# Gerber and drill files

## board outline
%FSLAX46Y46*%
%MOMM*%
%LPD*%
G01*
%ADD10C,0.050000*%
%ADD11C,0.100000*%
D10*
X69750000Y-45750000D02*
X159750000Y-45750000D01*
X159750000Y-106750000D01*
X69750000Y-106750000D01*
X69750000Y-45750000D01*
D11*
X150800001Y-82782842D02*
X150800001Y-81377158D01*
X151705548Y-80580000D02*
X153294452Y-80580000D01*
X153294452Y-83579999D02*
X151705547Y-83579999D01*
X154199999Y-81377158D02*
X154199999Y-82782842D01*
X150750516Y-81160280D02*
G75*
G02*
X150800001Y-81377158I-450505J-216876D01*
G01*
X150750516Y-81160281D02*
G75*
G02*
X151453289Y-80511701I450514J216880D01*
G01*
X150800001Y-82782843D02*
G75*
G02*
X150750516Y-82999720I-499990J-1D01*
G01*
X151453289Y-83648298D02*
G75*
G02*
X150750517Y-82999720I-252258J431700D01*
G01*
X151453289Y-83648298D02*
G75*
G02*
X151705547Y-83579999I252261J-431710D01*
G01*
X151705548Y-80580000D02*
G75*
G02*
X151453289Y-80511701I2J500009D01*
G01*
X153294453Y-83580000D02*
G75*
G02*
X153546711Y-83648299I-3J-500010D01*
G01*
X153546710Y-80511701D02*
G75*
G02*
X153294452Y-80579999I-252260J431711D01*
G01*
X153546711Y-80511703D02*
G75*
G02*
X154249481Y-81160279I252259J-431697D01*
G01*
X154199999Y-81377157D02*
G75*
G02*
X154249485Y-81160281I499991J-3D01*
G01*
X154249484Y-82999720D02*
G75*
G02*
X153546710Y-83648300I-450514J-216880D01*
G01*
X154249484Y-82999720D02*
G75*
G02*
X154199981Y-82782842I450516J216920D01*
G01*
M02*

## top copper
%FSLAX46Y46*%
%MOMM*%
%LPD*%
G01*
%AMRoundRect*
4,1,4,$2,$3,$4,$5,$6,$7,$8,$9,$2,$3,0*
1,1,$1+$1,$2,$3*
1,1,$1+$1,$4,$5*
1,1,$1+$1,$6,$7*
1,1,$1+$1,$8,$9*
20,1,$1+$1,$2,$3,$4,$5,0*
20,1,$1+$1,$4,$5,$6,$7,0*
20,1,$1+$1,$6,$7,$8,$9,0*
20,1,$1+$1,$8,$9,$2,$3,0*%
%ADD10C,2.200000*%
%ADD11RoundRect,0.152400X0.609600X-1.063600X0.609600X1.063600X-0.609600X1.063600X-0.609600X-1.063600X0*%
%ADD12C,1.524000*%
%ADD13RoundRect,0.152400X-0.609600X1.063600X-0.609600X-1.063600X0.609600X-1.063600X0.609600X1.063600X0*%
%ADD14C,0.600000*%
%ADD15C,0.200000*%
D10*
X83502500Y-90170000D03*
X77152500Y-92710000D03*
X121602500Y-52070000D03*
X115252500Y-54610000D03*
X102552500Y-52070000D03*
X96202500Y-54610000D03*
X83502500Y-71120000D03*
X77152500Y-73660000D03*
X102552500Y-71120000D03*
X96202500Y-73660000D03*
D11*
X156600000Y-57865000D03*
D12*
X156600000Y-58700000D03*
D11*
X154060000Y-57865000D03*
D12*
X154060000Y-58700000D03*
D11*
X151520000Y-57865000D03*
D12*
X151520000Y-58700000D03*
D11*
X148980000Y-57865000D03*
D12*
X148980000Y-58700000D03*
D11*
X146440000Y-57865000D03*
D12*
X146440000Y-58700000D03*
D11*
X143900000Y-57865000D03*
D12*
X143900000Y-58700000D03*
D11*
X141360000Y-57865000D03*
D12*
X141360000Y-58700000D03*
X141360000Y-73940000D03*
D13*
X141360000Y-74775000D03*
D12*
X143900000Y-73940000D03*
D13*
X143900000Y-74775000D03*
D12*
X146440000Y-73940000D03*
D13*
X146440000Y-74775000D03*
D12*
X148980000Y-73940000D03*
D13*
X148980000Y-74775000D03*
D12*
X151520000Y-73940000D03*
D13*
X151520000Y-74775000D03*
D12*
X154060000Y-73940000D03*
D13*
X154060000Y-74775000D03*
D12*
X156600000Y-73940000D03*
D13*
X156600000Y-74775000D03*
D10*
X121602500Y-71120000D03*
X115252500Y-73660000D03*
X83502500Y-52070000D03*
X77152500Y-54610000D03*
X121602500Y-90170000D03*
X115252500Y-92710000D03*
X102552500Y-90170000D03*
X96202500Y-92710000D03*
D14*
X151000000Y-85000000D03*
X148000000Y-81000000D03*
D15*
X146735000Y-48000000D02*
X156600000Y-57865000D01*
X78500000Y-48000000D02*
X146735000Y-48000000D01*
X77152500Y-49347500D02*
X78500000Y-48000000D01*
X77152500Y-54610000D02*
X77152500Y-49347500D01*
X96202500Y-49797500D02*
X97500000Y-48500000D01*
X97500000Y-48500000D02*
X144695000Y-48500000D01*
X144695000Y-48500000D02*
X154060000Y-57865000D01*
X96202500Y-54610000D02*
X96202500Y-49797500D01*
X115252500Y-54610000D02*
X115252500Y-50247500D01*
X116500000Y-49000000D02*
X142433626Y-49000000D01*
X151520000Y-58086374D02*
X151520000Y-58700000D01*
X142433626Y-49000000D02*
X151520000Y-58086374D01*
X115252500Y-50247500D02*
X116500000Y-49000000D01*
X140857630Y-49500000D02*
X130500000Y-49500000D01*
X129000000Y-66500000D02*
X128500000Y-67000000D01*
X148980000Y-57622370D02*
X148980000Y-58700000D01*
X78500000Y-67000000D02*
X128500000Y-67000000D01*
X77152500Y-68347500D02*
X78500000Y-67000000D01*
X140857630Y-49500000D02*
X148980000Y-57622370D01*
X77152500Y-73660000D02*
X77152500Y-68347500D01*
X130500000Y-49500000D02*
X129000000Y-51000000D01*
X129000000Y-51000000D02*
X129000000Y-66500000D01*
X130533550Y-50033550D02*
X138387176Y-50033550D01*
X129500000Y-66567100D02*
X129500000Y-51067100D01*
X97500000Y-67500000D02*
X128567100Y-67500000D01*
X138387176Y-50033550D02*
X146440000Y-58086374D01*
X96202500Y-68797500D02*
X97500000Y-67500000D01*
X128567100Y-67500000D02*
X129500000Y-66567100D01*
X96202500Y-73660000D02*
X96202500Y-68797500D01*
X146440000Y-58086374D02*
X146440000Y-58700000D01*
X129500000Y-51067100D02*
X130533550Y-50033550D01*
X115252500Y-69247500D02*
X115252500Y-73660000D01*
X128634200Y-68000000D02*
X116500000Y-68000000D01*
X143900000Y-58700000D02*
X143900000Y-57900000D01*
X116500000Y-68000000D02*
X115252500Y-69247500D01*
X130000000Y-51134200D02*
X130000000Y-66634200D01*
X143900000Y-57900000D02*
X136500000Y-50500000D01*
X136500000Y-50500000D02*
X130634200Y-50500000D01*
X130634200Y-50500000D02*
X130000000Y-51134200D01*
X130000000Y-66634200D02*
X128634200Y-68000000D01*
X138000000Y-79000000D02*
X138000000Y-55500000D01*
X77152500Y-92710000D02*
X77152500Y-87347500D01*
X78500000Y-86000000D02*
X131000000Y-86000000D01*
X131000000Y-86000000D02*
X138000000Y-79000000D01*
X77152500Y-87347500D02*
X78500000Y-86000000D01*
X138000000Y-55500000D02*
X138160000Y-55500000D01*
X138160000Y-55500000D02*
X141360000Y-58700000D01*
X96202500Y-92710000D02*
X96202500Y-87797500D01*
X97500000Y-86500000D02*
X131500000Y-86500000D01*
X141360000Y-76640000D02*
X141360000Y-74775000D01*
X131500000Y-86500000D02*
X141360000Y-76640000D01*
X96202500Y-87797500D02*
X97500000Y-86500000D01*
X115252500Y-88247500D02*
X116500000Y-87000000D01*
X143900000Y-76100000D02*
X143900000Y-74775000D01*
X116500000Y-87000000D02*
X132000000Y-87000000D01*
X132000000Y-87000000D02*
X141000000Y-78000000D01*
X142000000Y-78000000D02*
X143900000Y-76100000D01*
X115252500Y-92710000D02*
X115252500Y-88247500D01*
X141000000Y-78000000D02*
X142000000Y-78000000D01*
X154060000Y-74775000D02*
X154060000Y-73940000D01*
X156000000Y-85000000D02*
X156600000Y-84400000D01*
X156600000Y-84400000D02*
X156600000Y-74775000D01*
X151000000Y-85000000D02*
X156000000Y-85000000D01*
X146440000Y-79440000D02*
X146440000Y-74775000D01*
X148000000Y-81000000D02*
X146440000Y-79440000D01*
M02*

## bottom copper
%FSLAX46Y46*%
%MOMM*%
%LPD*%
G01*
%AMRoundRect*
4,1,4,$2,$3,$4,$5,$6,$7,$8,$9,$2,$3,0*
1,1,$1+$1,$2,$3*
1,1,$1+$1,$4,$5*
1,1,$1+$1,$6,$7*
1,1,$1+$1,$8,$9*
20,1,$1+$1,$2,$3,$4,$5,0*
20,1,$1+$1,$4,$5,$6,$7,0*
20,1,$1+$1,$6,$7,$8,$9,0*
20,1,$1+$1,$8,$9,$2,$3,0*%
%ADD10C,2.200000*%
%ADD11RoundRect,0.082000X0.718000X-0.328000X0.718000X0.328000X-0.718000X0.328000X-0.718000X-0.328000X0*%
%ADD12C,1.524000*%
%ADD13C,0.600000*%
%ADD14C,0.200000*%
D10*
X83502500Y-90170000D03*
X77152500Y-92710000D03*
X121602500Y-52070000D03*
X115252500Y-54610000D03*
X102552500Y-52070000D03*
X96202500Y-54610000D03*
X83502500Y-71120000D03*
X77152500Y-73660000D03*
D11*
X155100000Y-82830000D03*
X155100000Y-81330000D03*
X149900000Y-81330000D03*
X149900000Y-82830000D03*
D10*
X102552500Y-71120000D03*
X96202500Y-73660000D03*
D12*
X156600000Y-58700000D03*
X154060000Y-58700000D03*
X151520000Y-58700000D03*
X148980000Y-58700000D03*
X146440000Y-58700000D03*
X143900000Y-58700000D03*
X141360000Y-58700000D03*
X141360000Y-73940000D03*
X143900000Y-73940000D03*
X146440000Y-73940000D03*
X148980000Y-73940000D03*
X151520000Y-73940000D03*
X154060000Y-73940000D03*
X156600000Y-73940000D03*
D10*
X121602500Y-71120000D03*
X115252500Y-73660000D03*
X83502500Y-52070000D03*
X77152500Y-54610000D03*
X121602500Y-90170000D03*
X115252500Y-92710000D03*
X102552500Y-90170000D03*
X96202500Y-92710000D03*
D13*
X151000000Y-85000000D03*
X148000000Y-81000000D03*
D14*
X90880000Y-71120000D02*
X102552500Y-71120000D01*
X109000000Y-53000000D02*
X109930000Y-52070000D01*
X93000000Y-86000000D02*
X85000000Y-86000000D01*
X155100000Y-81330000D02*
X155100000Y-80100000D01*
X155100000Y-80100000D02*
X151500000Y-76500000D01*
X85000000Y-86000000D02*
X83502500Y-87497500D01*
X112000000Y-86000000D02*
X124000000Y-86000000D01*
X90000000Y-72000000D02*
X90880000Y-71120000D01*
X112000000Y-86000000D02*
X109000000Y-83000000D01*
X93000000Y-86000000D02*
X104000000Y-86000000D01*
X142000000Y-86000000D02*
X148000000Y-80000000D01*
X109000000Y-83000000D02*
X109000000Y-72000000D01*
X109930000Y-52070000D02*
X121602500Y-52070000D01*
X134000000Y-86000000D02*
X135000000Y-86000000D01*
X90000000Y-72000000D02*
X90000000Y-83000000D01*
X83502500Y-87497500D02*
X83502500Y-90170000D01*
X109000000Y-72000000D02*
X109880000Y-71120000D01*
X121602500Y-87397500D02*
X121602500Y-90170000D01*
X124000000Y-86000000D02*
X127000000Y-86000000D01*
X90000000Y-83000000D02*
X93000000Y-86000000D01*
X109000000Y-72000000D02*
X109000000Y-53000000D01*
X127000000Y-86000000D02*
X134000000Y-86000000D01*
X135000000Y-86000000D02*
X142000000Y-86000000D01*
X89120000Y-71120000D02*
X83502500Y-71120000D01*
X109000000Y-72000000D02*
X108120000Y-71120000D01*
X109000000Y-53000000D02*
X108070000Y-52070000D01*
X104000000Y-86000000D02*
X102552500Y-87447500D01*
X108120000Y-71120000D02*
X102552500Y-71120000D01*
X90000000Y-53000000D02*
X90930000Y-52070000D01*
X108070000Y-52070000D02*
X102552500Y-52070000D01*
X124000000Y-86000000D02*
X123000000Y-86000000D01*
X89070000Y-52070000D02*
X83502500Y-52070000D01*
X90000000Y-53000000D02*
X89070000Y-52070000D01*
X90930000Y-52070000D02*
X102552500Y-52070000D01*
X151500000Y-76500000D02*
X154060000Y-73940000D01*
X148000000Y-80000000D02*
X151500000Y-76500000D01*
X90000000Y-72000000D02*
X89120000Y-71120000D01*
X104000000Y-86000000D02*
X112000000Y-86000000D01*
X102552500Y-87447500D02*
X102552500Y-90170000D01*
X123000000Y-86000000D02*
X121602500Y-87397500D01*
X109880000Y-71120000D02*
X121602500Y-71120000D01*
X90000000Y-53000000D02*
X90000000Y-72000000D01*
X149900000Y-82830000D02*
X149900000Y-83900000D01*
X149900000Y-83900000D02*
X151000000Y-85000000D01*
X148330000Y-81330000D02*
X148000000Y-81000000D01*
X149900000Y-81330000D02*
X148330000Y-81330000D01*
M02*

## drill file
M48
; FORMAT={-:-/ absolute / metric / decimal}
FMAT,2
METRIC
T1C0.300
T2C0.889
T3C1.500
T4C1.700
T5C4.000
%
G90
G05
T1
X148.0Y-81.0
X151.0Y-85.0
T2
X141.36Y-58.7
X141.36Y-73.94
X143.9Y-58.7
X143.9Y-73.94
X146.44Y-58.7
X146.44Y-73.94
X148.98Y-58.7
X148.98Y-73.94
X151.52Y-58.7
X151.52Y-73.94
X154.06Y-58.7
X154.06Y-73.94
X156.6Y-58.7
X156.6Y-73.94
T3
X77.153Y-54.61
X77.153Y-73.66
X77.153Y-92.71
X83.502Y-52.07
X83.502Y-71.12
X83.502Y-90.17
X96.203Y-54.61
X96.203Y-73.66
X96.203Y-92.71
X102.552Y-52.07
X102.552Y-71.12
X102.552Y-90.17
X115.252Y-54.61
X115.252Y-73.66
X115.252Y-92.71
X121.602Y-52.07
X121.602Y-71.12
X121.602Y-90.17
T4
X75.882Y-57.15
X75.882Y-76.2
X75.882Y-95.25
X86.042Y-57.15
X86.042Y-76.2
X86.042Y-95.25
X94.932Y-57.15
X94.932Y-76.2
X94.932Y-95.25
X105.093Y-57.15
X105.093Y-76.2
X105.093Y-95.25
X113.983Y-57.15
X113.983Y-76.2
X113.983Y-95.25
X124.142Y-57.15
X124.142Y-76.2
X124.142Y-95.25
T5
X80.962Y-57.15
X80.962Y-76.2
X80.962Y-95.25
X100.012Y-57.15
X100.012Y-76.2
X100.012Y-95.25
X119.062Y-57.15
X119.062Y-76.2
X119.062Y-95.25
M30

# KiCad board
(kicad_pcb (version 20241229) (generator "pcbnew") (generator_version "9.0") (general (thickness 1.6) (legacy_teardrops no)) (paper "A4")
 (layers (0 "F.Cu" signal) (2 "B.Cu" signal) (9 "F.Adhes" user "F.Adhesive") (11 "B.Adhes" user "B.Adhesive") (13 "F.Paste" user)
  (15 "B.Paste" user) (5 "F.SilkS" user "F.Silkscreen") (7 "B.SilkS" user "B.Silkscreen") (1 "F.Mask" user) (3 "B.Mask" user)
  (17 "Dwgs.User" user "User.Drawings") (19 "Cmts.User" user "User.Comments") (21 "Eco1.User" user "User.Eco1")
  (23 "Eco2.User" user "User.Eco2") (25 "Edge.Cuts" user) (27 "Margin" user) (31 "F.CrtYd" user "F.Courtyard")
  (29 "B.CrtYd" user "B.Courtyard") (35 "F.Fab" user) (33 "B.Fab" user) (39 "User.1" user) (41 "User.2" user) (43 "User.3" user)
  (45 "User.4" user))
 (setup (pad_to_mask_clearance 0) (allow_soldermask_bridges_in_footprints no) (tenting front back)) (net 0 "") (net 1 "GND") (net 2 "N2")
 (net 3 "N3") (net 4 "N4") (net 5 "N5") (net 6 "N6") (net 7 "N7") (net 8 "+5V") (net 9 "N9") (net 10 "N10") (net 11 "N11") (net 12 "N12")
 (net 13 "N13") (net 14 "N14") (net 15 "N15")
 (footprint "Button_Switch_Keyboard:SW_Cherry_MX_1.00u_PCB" (layer "F.Cu") (at 83.5025 90.17)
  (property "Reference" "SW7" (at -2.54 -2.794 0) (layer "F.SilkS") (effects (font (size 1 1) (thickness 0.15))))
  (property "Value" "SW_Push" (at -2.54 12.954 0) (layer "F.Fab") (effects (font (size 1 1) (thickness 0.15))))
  (pad "" np_thru_hole circle (at -7.62 5.08) (size 1.7 1.7) (drill 1.7) (layers "*.Cu" "*.Mask"))
  (pad "" np_thru_hole circle (at -2.54 5.08) (size 4 4) (drill 4) (layers "*.Cu" "*.Mask"))
  (pad "" np_thru_hole circle (at 2.54 5.08) (size 1.7 1.7) (drill 1.7) (layers "*.Cu" "*.Mask"))
  (pad "1" thru_hole circle (at 0 0) (size 2.2 2.2) (drill 1.5) (layers "*.Cu" "*.Mask") (remove_unused_layers no) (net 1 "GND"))
  (pad "2" thru_hole circle (at -6.35 2.54) (size 2.2 2.2) (drill 1.5) (layers "*.Cu" "*.Mask") (remove_unused_layers no) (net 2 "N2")))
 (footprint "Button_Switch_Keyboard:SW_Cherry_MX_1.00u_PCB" (layer "F.Cu") (at 121.6025 52.07)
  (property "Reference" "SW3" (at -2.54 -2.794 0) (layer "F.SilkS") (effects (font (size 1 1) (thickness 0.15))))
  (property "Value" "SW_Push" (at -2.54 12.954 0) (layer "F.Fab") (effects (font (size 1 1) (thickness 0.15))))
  (pad "" np_thru_hole circle (at -7.62 5.08) (size 1.7 1.7) (drill 1.7) (layers "*.Cu" "*.Mask"))
  (pad "" np_thru_hole circle (at -2.54 5.08) (size 4 4) (drill 4) (layers "*.Cu" "*.Mask"))
  (pad "" np_thru_hole circle (at 2.54 5.08) (size 1.7 1.7) (drill 1.7) (layers "*.Cu" "*.Mask"))
  (pad "1" thru_hole circle (at 0 0) (size 2.2 2.2) (drill 1.5) (layers "*.Cu" "*.Mask") (remove_unused_layers no) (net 1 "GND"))
  (pad "2" thru_hole circle (at -6.35 2.54) (size 2.2 2.2) (drill 1.5) (layers "*.Cu" "*.Mask") (remove_unused_layers no) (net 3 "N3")))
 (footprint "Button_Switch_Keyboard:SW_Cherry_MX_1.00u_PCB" (layer "F.Cu") (at 102.5525 52.07)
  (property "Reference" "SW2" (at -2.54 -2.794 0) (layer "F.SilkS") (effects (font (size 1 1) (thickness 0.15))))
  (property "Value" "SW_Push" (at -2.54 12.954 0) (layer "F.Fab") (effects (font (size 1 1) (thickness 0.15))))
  (pad "" np_thru_hole circle (at -7.62 5.08) (size 1.7 1.7) (drill 1.7) (layers "*.Cu" "*.Mask"))
  (pad "" np_thru_hole circle (at -2.54 5.08) (size 4 4) (drill 4) (layers "*.Cu" "*.Mask"))
  (pad "" np_thru_hole circle (at 2.54 5.08) (size 1.7 1.7) (drill 1.7) (layers "*.Cu" "*.Mask"))
  (pad "1" thru_hole circle (at 0 0) (size 2.2 2.2) (drill 1.5) (layers "*.Cu" "*.Mask") (remove_unused_layers no) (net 1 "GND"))
  (pad "2" thru_hole circle (at -6.35 2.54) (size 2.2 2.2) (drill 1.5) (layers "*.Cu" "*.Mask") (remove_unused_layers no) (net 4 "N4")))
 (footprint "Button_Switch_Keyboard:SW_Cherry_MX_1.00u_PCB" (layer "F.Cu") (at 83.5025 71.12)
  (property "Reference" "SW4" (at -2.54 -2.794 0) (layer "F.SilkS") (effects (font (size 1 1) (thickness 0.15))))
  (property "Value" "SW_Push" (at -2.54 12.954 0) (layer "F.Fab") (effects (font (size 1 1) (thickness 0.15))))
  (pad "" np_thru_hole circle (at -7.62 5.08) (size 1.7 1.7) (drill 1.7) (layers "*.Cu" "*.Mask"))
  (pad "" np_thru_hole circle (at -2.54 5.08) (size 4 4) (drill 4) (layers "*.Cu" "*.Mask"))
  (pad "" np_thru_hole circle (at 2.54 5.08) (size 1.7 1.7) (drill 1.7) (layers "*.Cu" "*.Mask"))
  (pad "1" thru_hole circle (at 0 0) (size 2.2 2.2) (drill 1.5) (layers "*.Cu" "*.Mask") (remove_unused_layers no) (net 1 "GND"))
  (pad "2" thru_hole circle (at -6.35 2.54) (size 2.2 2.2) (drill 1.5) (layers "*.Cu" "*.Mask") (remove_unused_layers no) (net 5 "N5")))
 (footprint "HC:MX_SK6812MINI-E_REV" (layer "F.Cu") (at 152.5 77)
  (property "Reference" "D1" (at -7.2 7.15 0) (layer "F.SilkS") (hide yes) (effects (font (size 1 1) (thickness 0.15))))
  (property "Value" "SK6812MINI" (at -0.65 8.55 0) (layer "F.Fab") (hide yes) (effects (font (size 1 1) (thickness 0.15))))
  (fp_line (start -1.699999 5.782842) (end -1.699999 4.377158) (stroke (width 0.1) (type solid)) (layer "Edge.Cuts"))
  (fp_line (start -0.794452 3.58) (end 0.794452 3.58) (stroke (width 0.1) (type solid)) (layer "Edge.Cuts"))
  (fp_line (start 0.794452 6.579999) (end -0.794453 6.579999) (stroke (width 0.1) (type solid)) (layer "Edge.Cuts"))
  (fp_line (start 1.699999 4.377158) (end 1.699999 5.782842) (stroke (width 0.1) (type solid)) (layer "Edge.Cuts"))
  (fp_arc (start -1.749484 4.16028) (mid -1.712527 4.265932) (end -1.699999 4.377158) (stroke (width 0.1) (type solid)) (layer "Edge.Cuts"))
  (fp_arc (start -1.749484 4.160281) (mid -1.638072 3.575965) (end -1.046711 3.511701) (stroke (width 0.1) (type solid)) (layer "Edge.Cuts"))
  (fp_arc (start -1.699999 5.782843) (mid -1.712527 5.894068) (end -1.749484 5.99972) (stroke (width 0.1) (type solid)) (layer "Edge.Cuts"))
  (fp_arc (start -1.046711 6.648298) (mid -1.638071 6.584034) (end -1.749484 5.99972) (stroke (width 0.1) (type solid)) (layer "Edge.Cuts"))
  (fp_arc (start -1.046711 6.648298) (mid -0.925123 6.597376) (end -0.794453 6.579999) (stroke (width 0.1) (type solid)) (layer "Edge.Cuts"))
  (fp_arc (start -0.794452 3.58) (mid -0.925123 3.562623) (end -1.046711 3.511701) (stroke (width 0.1) (type solid)) (layer "Edge.Cuts"))
  (fp_arc (start 0.794453 6.58) (mid 0.925123 6.597377) (end 1.046711 6.648299) (stroke (width 0.1) (type solid)) (layer "Edge.Cuts"))
  (fp_arc (start 1.04671 3.511701) (mid 0.925122 3.562623) (end 0.794452 3.58) (stroke (width 0.1) (type solid)) (layer "Edge.Cuts"))
  (fp_arc (start 1.046711 3.511703) (mid 1.63807 3.575966) (end 1.749484 4.16028) (stroke (width 0.1) (type solid)) (layer "Edge.Cuts"))
  (fp_arc (start 1.699999 4.377157) (mid 1.712527 4.265932) (end 1.749484 4.16028) (stroke (width 0.1) (type solid)) (layer "Edge.Cuts"))
  (fp_arc (start 1.749484 5.99972) (mid 1.638071 6.584035) (end 1.046711 6.648299) (stroke (width 0.1) (type solid)) (layer "Edge.Cuts"))
  (fp_arc (start 1.749484 5.99972) (mid 1.712527 5.894068) (end 1.699999 5.782842) (stroke (width 0.1) (type solid)) (layer "Edge.Cuts"))
  (pad "1" smd roundrect (at 2.6 5.83 90) (size 0.82 1.6) (layers "B.Cu" "B.Mask" "B.Paste") (roundrect_rratio 0.1) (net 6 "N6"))
  (pad "2" smd roundrect (at 2.6 4.33 90) (size 0.82 1.6) (layers "B.Cu" "B.Mask" "B.Paste") (roundrect_rratio 0.1) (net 1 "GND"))
  (pad "3" smd roundrect (at -2.6 4.33 90) (size 0.82 1.6) (layers "B.Cu" "B.Mask" "B.Paste") (roundrect_rratio 0.1) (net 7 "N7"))
  (pad "4" smd roundrect (at -2.6 5.83 90) (size 0.82 1.6) (layers "B.Cu" "B.Mask" "B.Paste") (roundrect_rratio 0.1) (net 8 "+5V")))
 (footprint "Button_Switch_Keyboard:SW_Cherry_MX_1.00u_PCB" (layer "F.Cu") (at 102.5525 71.12)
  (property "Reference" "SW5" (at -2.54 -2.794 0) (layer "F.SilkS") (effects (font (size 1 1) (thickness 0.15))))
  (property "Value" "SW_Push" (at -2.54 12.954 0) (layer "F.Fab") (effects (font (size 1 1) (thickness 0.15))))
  (pad "" np_thru_hole circle (at -7.62 5.08) (size 1.7 1.7) (drill 1.7) (layers "*.Cu" "*.Mask"))
  (pad "" np_thru_hole circle (at -2.54 5.08) (size 4 4) (drill 4) (layers "*.Cu" "*.Mask"))
  (pad "" np_thru_hole circle (at 2.54 5.08) (size 1.7 1.7) (drill 1.7) (layers "*.Cu" "*.Mask"))
  (pad "1" thru_hole circle (at 0 0) (size 2.2 2.2) (drill 1.5) (layers "*.Cu" "*.Mask") (remove_unused_layers no) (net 1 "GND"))
  (pad "2" thru_hole circle (at -6.35 2.54) (size 2.2 2.2) (drill 1.5) (layers "*.Cu" "*.Mask") (remove_unused_layers no) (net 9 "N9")))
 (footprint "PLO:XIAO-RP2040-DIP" (layer "F.Cu") (at 148.98 66.32 -90)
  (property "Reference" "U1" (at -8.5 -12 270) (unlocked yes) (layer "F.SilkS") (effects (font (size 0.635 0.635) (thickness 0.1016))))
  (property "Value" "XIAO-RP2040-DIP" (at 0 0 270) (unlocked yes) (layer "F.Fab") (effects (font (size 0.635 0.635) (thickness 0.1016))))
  (pad "1" smd roundrect (at -8.455 -7.62 90) (size 2.432 1.524) (layers "F.Cu" "F.Mask") (roundrect_rratio 0.1) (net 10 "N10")
   (thermal_bridge_angle 45))
  (pad "1" thru_hole circle (at -7.62 -7.62 90) (size 1.524 1.524) (drill 0.889) (layers "*.Cu" "*.Mask") (remove_unused_layers no)
   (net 10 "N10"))
  (pad "2" smd roundrect (at -8.455 -5.08 90) (size 2.432 1.524) (layers "F.Cu" "F.Mask") (roundrect_rratio 0.1) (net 4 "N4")
   (thermal_bridge_angle 45))
  (pad "2" thru_hole circle (at -7.62 -5.08 90) (size 1.524 1.524) (drill 0.889) (layers "*.Cu" "*.Mask") (remove_unused_layers no)
   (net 4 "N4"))
  (pad "3" smd roundrect (at -8.455 -2.54 90) (size 2.432 1.524) (layers "F.Cu" "F.Mask") (roundrect_rratio 0.1) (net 3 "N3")
   (thermal_bridge_angle 45))
  (pad "3" thru_hole circle (at -7.62 -2.54 90) (size 1.524 1.524) (drill 0.889) (layers "*.Cu" "*.Mask") (remove_unused_layers no)
   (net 3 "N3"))
  (pad "4" smd roundrect (at -8.455 0 90) (size 2.432 1.524) (layers "F.Cu" "F.Mask") (roundrect_rratio 0.1) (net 5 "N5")
   (thermal_bridge_angle 45))
  (pad "4" thru_hole circle (at -7.62 0 90) (size 1.524 1.524) (drill 0.889) (layers "*.Cu" "*.Mask") (remove_unused_layers no) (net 5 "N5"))
  (pad "5" smd roundrect (at -8.455 2.54 90) (size 2.432 1.524) (layers "F.Cu" "F.Mask") (roundrect_rratio 0.1) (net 9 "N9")
   (thermal_bridge_angle 45))
  (pad "5" thru_hole circle (at -7.62 2.54 90) (size 1.524 1.524) (drill 0.889) (layers "*.Cu" "*.Mask") (remove_unused_layers no)
   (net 9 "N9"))
  (pad "6" smd roundrect (at -8.455 5.08 90) (size 2.432 1.524) (layers "F.Cu" "F.Mask") (roundrect_rratio 0.1) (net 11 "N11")
   (thermal_bridge_angle 45))
  (pad "6" thru_hole circle (at -7.62 5.08 90) (size 1.524 1.524) (drill 0.889) (layers "*.Cu" "*.Mask") (remove_unused_layers no)
   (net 11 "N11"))
  (pad "7" smd roundrect (at -8.455 7.62 90) (size 2.432 1.524) (layers "F.Cu" "F.Mask") (roundrect_rratio 0.1) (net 2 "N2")
   (thermal_bridge_angle 45))
  (pad "7" thru_hole circle (at -7.62 7.62 90) (size 1.524 1.524) (drill 0.889) (layers "*.Cu" "*.Mask") (remove_unused_layers no)
   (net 2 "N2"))
  (pad "8" thru_hole circle (at 7.62 7.62 270) (size 1.524 1.524) (drill 0.889) (layers "*.Cu" "*.Mask") (remove_unused_layers no)
   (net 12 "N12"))
  (pad "8" smd roundrect (at 8.455 7.62 270) (size 2.432 1.524) (layers "F.Cu" "F.Mask") (roundrect_rratio 0.1) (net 12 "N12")
   (thermal_bridge_angle 45))
  (pad "9" thru_hole circle (at 7.62 5.08 270) (size 1.524 1.524) (drill 0.889) (layers "*.Cu" "*.Mask") (remove_unused_layers no)
   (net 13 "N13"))
  (pad "9" smd roundrect (at 8.455 5.08 270) (size 2.432 1.524) (layers "F.Cu" "F.Mask") (roundrect_rratio 0.1) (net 13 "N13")
   (thermal_bridge_angle 45))
  (pad "10" thru_hole circle (at 7.62 2.54 270) (size 1.524 1.524) (drill 0.889) (layers "*.Cu" "*.Mask") (remove_unused_layers no)
   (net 7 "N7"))
  (pad "10" smd roundrect (at 8.455 2.54 270) (size 2.432 1.524) (layers "F.Cu" "F.Mask") (roundrect_rratio 0.1) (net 7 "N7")
   (thermal_bridge_angle 45))
  (pad "11" thru_hole circle (at 7.62 0 270) (size 1.524 1.524) (drill 0.889) (layers "*.Cu" "*.Mask") (remove_unused_layers no)
   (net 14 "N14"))
  (pad "11" smd roundrect (at 8.455 0 270) (size 2.432 1.524) (layers "F.Cu" "F.Mask") (roundrect_rratio 0.1) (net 14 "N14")
   (thermal_bridge_angle 45))
  (pad "12" thru_hole circle (at 7.62 -2.54 270) (size 1.524 1.524) (drill 0.889) (layers "*.Cu" "*.Mask") (remove_unused_layers no)
   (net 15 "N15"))
  (pad "12" smd roundrect (at 8.455 -2.54 270) (size 2.432 1.524) (layers "F.Cu" "F.Mask") (roundrect_rratio 0.1) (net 15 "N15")
   (thermal_bridge_angle 45))
  (pad "13" thru_hole circle (at 7.62 -5.08 270) (size 1.524 1.524) (drill 0.889) (layers "*.Cu" "*.Mask") (remove_unused_layers no)
   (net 1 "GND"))
  (pad "13" smd roundrect (at 8.455 -5.08 270) (size 2.432 1.524) (layers "F.Cu" "F.Mask") (roundrect_rratio 0.1) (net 1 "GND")
   (thermal_bridge_angle 45))
  (pad "14" thru_hole circle (at 7.62 -7.62 270) (size 1.524 1.524) (drill 0.889) (layers "*.Cu" "*.Mask") (remove_unused_layers no)
   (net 8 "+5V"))
  (pad "14" smd roundrect (at 8.455 -7.62 270) (size 2.432 1.524) (layers "F.Cu" "F.Mask") (roundrect_rratio 0.1) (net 8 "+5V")
   (thermal_bridge_angle 45)))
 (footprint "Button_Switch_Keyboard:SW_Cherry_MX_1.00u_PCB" (layer "F.Cu") (at 121.6025 71.12)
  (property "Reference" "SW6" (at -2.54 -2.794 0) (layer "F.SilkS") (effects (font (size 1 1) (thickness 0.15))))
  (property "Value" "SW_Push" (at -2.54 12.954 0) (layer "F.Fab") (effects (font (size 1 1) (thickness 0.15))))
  (pad "" np_thru_hole circle (at -7.62 5.08) (size 1.7 1.7) (drill 1.7) (layers "*.Cu" "*.Mask"))
  (pad "" np_thru_hole circle (at -2.54 5.08) (size 4 4) (drill 4) (layers "*.Cu" "*.Mask"))
  (pad "" np_thru_hole circle (at 2.54 5.08) (size 1.7 1.7) (drill 1.7) (layers "*.Cu" "*.Mask"))
  (pad "1" thru_hole circle (at 0 0) (size 2.2 2.2) (drill 1.5) (layers "*.Cu" "*.Mask") (remove_unused_layers no) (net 1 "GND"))
  (pad "2" thru_hole circle (at -6.35 2.54) (size 2.2 2.2) (drill 1.5) (layers "*.Cu" "*.Mask") (remove_unused_layers no) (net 11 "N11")))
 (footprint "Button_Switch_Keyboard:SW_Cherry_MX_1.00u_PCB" (layer "F.Cu") (at 83.5025 52.07)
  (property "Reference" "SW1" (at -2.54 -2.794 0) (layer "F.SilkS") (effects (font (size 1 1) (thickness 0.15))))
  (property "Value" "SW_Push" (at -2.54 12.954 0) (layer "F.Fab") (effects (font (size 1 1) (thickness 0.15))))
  (pad "" np_thru_hole circle (at -7.62 5.08) (size 1.7 1.7) (drill 1.7) (layers "*.Cu" "*.Mask"))
  (pad "" np_thru_hole circle (at -2.54 5.08) (size 4 4) (drill 4) (layers "*.Cu" "*.Mask"))
  (pad "" np_thru_hole circle (at 2.54 5.08) (size 1.7 1.7) (drill 1.7) (layers "*.Cu" "*.Mask"))
  (pad "1" thru_hole circle (at 0 0) (size 2.2 2.2) (drill 1.5) (layers "*.Cu" "*.Mask") (remove_unused_layers no) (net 1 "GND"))
  (pad "2" thru_hole circle (at -6.35 2.54) (size 2.2 2.2) (drill 1.5) (layers "*.Cu" "*.Mask") (remove_unused_layers no) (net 10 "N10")))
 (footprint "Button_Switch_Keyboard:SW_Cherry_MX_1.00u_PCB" (layer "F.Cu") (at 121.6025 90.17)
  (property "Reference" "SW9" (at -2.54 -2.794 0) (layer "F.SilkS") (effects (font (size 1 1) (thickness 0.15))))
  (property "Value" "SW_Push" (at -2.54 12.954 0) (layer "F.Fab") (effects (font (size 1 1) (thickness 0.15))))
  (pad "" np_thru_hole circle (at -7.62 5.08) (size 1.7 1.7) (drill 1.7) (layers "*.Cu" "*.Mask"))
  (pad "" np_thru_hole circle (at -2.54 5.08) (size 4 4) (drill 4) (layers "*.Cu" "*.Mask"))
  (pad "" np_thru_hole circle (at 2.54 5.08) (size 1.7 1.7) (drill 1.7) (layers "*.Cu" "*.Mask"))
  (pad "1" thru_hole circle (at 0 0) (size 2.2 2.2) (drill 1.5) (layers "*.Cu" "*.Mask") (remove_unused_layers no) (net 1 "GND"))
  (pad "2" thru_hole circle (at -6.35 2.54) (size 2.2 2.2) (drill 1.5) (layers "*.Cu" "*.Mask") (remove_unused_layers no) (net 13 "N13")))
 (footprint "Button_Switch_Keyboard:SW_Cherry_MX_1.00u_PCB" (layer "F.Cu") (at 102.5525 90.17)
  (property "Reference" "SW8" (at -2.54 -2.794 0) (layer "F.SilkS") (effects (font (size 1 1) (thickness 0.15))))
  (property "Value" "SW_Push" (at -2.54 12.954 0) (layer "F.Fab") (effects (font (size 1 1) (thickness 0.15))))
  (pad "" np_thru_hole circle (at -7.62 5.08) (size 1.7 1.7) (drill 1.7) (layers "*.Cu" "*.Mask"))
  (pad "" np_thru_hole circle (at -2.54 5.08) (size 4 4) (drill 4) (layers "*.Cu" "*.Mask"))
  (pad "" np_thru_hole circle (at 2.54 5.08) (size 1.7 1.7) (drill 1.7) (layers "*.Cu" "*.Mask"))
  (pad "1" thru_hole circle (at 0 0) (size 2.2 2.2) (drill 1.5) (layers "*.Cu" "*.Mask") (remove_unused_layers no) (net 1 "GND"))
  (pad "2" thru_hole circle (at -6.35 2.54) (size 2.2 2.2) (drill 1.5) (layers "*.Cu" "*.Mask") (remove_unused_layers no) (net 12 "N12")))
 (gr_rect (start 69.75 45.75) (end 159.75 106.75) (stroke (width 0.05) (type default)) (fill no) (layer "Edge.Cuts"))
 (segment (start 146.735 48) (end 156.6 57.865) (width 0.2) (layer "F.Cu") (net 10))
 (segment (start 78.5 48) (end 146.735 48) (width 0.2) (layer "F.Cu") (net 10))
 (segment (start 77.1525 49.3475) (end 78.5 48) (width 0.2) (layer "F.Cu") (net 10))
 (segment (start 77.1525 54.61) (end 77.1525 49.3475) (width 0.2) (layer "F.Cu") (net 10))
 (segment (start 96.2025 49.7975) (end 97.5 48.5) (width 0.2) (layer "F.Cu") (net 4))
 (segment (start 97.5 48.5) (end 144.695 48.5) (width 0.2) (layer "F.Cu") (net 4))
 (segment (start 144.695 48.5) (end 154.06 57.865) (width 0.2) (layer "F.Cu") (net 4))
 (segment (start 96.2025 54.61) (end 96.2025 49.7975) (width 0.2) (layer "F.Cu") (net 4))
 (segment (start 115.2525 54.61) (end 115.2525 50.2475) (width 0.2) (layer "F.Cu") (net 3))
 (segment (start 116.5 49) (end 142.433626 49) (width 0.2) (layer "F.Cu") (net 3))
 (segment (start 151.52 58.086374) (end 151.52 58.7) (width 0.2) (layer "F.Cu") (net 3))
 (segment (start 142.433626 49) (end 151.52 58.086374) (width 0.2) (layer "F.Cu") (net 3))
 (segment (start 115.2525 50.2475) (end 116.5 49) (width 0.2) (layer "F.Cu") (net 3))
 (segment (start 140.85763 49.5) (end 130.5 49.5) (width 0.2) (layer "F.Cu") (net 5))
 (segment (start 129 66.5) (end 128.5 67) (width 0.2) (layer "F.Cu") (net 5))
 (segment (start 148.98 57.62237) (end 148.98 58.7) (width 0.2) (layer "F.Cu") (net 5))
 (segment (start 78.5 67) (end 128.5 67) (width 0.2) (layer "F.Cu") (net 5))
 (segment (start 77.1525 68.3475) (end 78.5 67) (width 0.2) (layer "F.Cu") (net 5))
 (segment (start 140.85763 49.5) (end 148.98 57.62237) (width 0.2) (layer "F.Cu") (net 5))
 (segment (start 77.1525 73.66) (end 77.1525 68.3475) (width 0.2) (layer "F.Cu") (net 5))
 (segment (start 130.5 49.5) (end 129 51) (width 0.2) (layer "F.Cu") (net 5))
 (segment (start 129 51) (end 129 66.5) (width 0.2) (layer "F.Cu") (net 5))
 (segment (start 130.53355 50.03355) (end 138.387176 50.03355) (width 0.2) (layer "F.Cu") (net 9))
 (segment (start 129.5 66.5671) (end 129.5 51.0671) (width 0.2) (layer "F.Cu") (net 9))
 (segment (start 97.5 67.5) (end 128.5671 67.5) (width 0.2) (layer "F.Cu") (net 9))
 (segment (start 138.387176 50.03355) (end 146.44 58.086374) (width 0.2) (layer "F.Cu") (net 9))
 (segment (start 96.2025 68.7975) (end 97.5 67.5) (width 0.2) (layer "F.Cu") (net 9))
 (segment (start 128.5671 67.5) (end 129.5 66.5671) (width 0.2) (layer "F.Cu") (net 9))
 (segment (start 96.2025 73.66) (end 96.2025 68.7975) (width 0.2) (layer "F.Cu") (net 9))
 (segment (start 146.44 58.086374) (end 146.44 58.7) (width 0.2) (layer "F.Cu") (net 9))
 (segment (start 129.5 51.0671) (end 130.53355 50.03355) (width 0.2) (layer "F.Cu") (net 9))
 (segment (start 115.2525 69.2475) (end 115.2525 73.66) (width 0.2) (layer "F.Cu") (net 11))
 (segment (start 128.6342 68) (end 116.5 68) (width 0.2) (layer "F.Cu") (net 11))
 (segment (start 143.9 58.7) (end 143.9 57.9) (width 0.2) (layer "F.Cu") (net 11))
 (segment (start 116.5 68) (end 115.2525 69.2475) (width 0.2) (layer "F.Cu") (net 11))
 (segment (start 130 51.1342) (end 130 66.6342) (width 0.2) (layer "F.Cu") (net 11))
 (segment (start 143.9 57.9) (end 136.5 50.5) (width 0.2) (layer "F.Cu") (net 11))
 (segment (start 136.5 50.5) (end 130.6342 50.5) (width 0.2) (layer "F.Cu") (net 11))
 (segment (start 130.6342 50.5) (end 130 51.1342) (width 0.2) (layer "F.Cu") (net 11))
 (segment (start 130 66.6342) (end 128.6342 68) (width 0.2) (layer "F.Cu") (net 11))
 (segment (start 138 79) (end 138 55.5) (width 0.2) (layer "F.Cu") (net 2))
 (segment (start 77.1525 92.71) (end 77.1525 87.3475) (width 0.2) (layer "F.Cu") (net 2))
 (segment (start 78.5 86) (end 131 86) (width 0.2) (layer "F.Cu") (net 2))
 (segment (start 131 86) (end 138 79) (width 0.2) (layer "F.Cu") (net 2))
 (segment (start 77.1525 87.3475) (end 78.5 86) (width 0.2) (layer "F.Cu") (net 2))
 (segment (start 138 55.5) (end 138.16 55.5) (width 0.2) (layer "F.Cu") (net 2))
 (segment (start 138.16 55.5) (end 141.36 58.7) (width 0.2) (layer "F.Cu") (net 2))
 (segment (start 96.2025 92.71) (end 96.2025 87.7975) (width 0.2) (layer "F.Cu") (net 12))
 (segment (start 97.5 86.5) (end 131.5 86.5) (width 0.2) (layer "F.Cu") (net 12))
 (segment (start 141.36 76.64) (end 141.36 74.775) (width 0.2) (layer "F.Cu") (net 12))
 (segment (start 131.5 86.5) (end 141.36 76.64) (width 0.2) (layer "F.Cu") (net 12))
 (segment (start 96.2025 87.7975) (end 97.5 86.5) (width 0.2) (layer "F.Cu") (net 12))
 (segment (start 115.2525 88.2475) (end 116.5 87) (width 0.2) (layer "F.Cu") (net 13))
 (segment (start 143.9 76.1) (end 143.9 74.775) (width 0.2) (layer "F.Cu") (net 13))
 (segment (start 116.5 87) (end 132 87) (width 0.2) (layer "F.Cu") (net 13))
 (segment (start 132 87) (end 141 78) (width 0.2) (layer "F.Cu") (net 13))
 (segment (start 142 78) (end 143.9 76.1) (width 0.2) (layer "F.Cu") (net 13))
 (segment (start 115.2525 92.71) (end 115.2525 88.2475) (width 0.2) (layer "F.Cu") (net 13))
 (segment (start 141 78) (end 142 78) (width 0.2) (layer "F.Cu") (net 13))
 (segment (start 154.06 74.775) (end 154.06 73.94) (width 0.2) (layer "F.Cu") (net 1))
 (segment (start 90.88 71.12) (end 102.5525 71.12) (width 0.2) (layer "B.Cu") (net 1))
 (segment (start 109 53) (end 109.93 52.07) (width 0.2) (layer "B.Cu") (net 1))
 (segment (start 93 86) (end 85 86) (width 0.2) (layer "B.Cu") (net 1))
 (segment (start 155.1 81.33) (end 155.1 80.1) (width 0.2) (layer "B.Cu") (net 1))
 (segment (start 155.1 80.1) (end 151.5 76.5) (width 0.2) (layer "B.Cu") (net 1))
 (segment (start 85 86) (end 83.5025 87.4975) (width 0.2) (layer "B.Cu") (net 1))
 (segment (start 112 86) (end 124 86) (width 0.2) (layer "B.Cu") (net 1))
 (segment (start 90 72) (end 90.88 71.12) (width 0.2) (layer "B.Cu") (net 1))
 (segment (start 112 86) (end 109 83) (width 0.2) (layer "B.Cu") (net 1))
 (segment (start 93 86) (end 104 86) (width 0.2) (layer "B.Cu") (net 1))
 (segment (start 142 86) (end 148 80) (width 0.2) (layer "B.Cu") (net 1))
 (segment (start 109 83) (end 109 72) (width 0.2) (layer "B.Cu") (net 1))
 (segment (start 109.93 52.07) (end 121.6025 52.07) (width 0.2) (layer "B.Cu") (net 1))
 (segment (start 134 86) (end 135 86) (width 0.2) (layer "B.Cu") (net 1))
 (segment (start 90 72) (end 90 83) (width 0.2) (layer "B.Cu") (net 1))
 (segment (start 83.5025 87.4975) (end 83.5025 90.17) (width 0.2) (layer "B.Cu") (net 1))
 (segment (start 109 72) (end 109.88 71.12) (width 0.2) (layer "B.Cu") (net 1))
 (segment (start 121.6025 87.3975) (end 121.6025 90.17) (width 0.2) (layer "B.Cu") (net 1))
 (segment (start 124 86) (end 127 86) (width 0.2) (layer "B.Cu") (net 1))
 (segment (start 90 83) (end 93 86) (width 0.2) (layer "B.Cu") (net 1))
 (segment (start 109 72) (end 109 53) (width 0.2) (layer "B.Cu") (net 1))
 (segment (start 127 86) (end 134 86) (width 0.2) (layer "B.Cu") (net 1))
 (segment (start 135 86) (end 142 86) (width 0.2) (layer "B.Cu") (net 1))
 (segment (start 89.12 71.12) (end 83.5025 71.12) (width 0.2) (layer "B.Cu") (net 1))
 (segment (start 109 72) (end 108.12 71.12) (width 0.2) (layer "B.Cu") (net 1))
 (segment (start 109 53) (end 108.07 52.07) (width 0.2) (layer "B.Cu") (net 1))
 (segment (start 104 86) (end 102.5525 87.4475) (width 0.2) (layer "B.Cu") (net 1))
 (segment (start 108.12 71.12) (end 102.5525 71.12) (width 0.2) (layer "B.Cu") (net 1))
 (segment (start 90 53) (end 90.93 52.07) (width 0.2) (layer "B.Cu") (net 1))
 (segment (start 108.07 52.07) (end 102.5525 52.07) (width 0.2) (layer "B.Cu") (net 1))
 (segment (start 124 86) (end 123 86) (width 0.2) (layer "B.Cu") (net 1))
 (segment (start 89.07 52.07) (end 83.5025 52.07) (width 0.2) (layer "B.Cu") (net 1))
 (segment (start 90 53) (end 89.07 52.07) (width 0.2) (layer "B.Cu") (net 1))
 (segment (start 90.93 52.07) (end 102.5525 52.07) (width 0.2) (layer "B.Cu") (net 1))
 (segment (start 151.5 76.5) (end 154.06 73.94) (width 0.2) (layer "B.Cu") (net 1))
 (segment (start 148 80) (end 151.5 76.5) (width 0.2) (layer "B.Cu") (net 1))
 (segment (start 90 72) (end 89.12 71.12) (width 0.2) (layer "B.Cu") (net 1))
 (segment (start 104 86) (end 112 86) (width 0.2) (layer "B.Cu") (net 1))
 (segment (start 102.5525 87.4475) (end 102.5525 90.17) (width 0.2) (layer "B.Cu") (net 1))
 (segment (start 123 86) (end 121.6025 87.3975) (width 0.2) (layer "B.Cu") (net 1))
 (segment (start 109.88 71.12) (end 121.6025 71.12) (width 0.2) (layer "B.Cu") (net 1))
 (segment (start 90 53) (end 90 72) (width 0.2) (layer "B.Cu") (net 1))
 (segment (start 156 85) (end 156.6 84.4) (width 0.2) (layer "F.Cu") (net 8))
 (segment (start 156.6 84.4) (end 156.6 74.775) (width 0.2) (layer "F.Cu") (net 8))
 (segment (start 151 85) (end 156 85) (width 0.2) (layer "F.Cu") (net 8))
 (via (at 151 85) (size 0.6) (drill 0.3) (layers "F.Cu" "B.Cu") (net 8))
 (segment (start 149.9 82.83) (end 149.9 83.9) (width 0.2) (layer "B.Cu") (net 8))
 (segment (start 149.9 83.9) (end 151 85) (width 0.2) (layer "B.Cu") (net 8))
 (segment (start 146.44 79.44) (end 146.44 74.775) (width 0.2) (layer "F.Cu") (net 7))
 (segment (start 148 81) (end 146.44 79.44) (width 0.2) (layer "F.Cu") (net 7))
 (via (at 148 81) (size 0.6) (drill 0.3) (layers "F.Cu" "B.Cu") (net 7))
 (segment (start 148.33 81.33) (end 148 81) (width 0.2) (layer "B.Cu") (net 7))
 (segment (start 149.9 81.33) (end 148.33 81.33) (width 0.2) (layer "B.Cu") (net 7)))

